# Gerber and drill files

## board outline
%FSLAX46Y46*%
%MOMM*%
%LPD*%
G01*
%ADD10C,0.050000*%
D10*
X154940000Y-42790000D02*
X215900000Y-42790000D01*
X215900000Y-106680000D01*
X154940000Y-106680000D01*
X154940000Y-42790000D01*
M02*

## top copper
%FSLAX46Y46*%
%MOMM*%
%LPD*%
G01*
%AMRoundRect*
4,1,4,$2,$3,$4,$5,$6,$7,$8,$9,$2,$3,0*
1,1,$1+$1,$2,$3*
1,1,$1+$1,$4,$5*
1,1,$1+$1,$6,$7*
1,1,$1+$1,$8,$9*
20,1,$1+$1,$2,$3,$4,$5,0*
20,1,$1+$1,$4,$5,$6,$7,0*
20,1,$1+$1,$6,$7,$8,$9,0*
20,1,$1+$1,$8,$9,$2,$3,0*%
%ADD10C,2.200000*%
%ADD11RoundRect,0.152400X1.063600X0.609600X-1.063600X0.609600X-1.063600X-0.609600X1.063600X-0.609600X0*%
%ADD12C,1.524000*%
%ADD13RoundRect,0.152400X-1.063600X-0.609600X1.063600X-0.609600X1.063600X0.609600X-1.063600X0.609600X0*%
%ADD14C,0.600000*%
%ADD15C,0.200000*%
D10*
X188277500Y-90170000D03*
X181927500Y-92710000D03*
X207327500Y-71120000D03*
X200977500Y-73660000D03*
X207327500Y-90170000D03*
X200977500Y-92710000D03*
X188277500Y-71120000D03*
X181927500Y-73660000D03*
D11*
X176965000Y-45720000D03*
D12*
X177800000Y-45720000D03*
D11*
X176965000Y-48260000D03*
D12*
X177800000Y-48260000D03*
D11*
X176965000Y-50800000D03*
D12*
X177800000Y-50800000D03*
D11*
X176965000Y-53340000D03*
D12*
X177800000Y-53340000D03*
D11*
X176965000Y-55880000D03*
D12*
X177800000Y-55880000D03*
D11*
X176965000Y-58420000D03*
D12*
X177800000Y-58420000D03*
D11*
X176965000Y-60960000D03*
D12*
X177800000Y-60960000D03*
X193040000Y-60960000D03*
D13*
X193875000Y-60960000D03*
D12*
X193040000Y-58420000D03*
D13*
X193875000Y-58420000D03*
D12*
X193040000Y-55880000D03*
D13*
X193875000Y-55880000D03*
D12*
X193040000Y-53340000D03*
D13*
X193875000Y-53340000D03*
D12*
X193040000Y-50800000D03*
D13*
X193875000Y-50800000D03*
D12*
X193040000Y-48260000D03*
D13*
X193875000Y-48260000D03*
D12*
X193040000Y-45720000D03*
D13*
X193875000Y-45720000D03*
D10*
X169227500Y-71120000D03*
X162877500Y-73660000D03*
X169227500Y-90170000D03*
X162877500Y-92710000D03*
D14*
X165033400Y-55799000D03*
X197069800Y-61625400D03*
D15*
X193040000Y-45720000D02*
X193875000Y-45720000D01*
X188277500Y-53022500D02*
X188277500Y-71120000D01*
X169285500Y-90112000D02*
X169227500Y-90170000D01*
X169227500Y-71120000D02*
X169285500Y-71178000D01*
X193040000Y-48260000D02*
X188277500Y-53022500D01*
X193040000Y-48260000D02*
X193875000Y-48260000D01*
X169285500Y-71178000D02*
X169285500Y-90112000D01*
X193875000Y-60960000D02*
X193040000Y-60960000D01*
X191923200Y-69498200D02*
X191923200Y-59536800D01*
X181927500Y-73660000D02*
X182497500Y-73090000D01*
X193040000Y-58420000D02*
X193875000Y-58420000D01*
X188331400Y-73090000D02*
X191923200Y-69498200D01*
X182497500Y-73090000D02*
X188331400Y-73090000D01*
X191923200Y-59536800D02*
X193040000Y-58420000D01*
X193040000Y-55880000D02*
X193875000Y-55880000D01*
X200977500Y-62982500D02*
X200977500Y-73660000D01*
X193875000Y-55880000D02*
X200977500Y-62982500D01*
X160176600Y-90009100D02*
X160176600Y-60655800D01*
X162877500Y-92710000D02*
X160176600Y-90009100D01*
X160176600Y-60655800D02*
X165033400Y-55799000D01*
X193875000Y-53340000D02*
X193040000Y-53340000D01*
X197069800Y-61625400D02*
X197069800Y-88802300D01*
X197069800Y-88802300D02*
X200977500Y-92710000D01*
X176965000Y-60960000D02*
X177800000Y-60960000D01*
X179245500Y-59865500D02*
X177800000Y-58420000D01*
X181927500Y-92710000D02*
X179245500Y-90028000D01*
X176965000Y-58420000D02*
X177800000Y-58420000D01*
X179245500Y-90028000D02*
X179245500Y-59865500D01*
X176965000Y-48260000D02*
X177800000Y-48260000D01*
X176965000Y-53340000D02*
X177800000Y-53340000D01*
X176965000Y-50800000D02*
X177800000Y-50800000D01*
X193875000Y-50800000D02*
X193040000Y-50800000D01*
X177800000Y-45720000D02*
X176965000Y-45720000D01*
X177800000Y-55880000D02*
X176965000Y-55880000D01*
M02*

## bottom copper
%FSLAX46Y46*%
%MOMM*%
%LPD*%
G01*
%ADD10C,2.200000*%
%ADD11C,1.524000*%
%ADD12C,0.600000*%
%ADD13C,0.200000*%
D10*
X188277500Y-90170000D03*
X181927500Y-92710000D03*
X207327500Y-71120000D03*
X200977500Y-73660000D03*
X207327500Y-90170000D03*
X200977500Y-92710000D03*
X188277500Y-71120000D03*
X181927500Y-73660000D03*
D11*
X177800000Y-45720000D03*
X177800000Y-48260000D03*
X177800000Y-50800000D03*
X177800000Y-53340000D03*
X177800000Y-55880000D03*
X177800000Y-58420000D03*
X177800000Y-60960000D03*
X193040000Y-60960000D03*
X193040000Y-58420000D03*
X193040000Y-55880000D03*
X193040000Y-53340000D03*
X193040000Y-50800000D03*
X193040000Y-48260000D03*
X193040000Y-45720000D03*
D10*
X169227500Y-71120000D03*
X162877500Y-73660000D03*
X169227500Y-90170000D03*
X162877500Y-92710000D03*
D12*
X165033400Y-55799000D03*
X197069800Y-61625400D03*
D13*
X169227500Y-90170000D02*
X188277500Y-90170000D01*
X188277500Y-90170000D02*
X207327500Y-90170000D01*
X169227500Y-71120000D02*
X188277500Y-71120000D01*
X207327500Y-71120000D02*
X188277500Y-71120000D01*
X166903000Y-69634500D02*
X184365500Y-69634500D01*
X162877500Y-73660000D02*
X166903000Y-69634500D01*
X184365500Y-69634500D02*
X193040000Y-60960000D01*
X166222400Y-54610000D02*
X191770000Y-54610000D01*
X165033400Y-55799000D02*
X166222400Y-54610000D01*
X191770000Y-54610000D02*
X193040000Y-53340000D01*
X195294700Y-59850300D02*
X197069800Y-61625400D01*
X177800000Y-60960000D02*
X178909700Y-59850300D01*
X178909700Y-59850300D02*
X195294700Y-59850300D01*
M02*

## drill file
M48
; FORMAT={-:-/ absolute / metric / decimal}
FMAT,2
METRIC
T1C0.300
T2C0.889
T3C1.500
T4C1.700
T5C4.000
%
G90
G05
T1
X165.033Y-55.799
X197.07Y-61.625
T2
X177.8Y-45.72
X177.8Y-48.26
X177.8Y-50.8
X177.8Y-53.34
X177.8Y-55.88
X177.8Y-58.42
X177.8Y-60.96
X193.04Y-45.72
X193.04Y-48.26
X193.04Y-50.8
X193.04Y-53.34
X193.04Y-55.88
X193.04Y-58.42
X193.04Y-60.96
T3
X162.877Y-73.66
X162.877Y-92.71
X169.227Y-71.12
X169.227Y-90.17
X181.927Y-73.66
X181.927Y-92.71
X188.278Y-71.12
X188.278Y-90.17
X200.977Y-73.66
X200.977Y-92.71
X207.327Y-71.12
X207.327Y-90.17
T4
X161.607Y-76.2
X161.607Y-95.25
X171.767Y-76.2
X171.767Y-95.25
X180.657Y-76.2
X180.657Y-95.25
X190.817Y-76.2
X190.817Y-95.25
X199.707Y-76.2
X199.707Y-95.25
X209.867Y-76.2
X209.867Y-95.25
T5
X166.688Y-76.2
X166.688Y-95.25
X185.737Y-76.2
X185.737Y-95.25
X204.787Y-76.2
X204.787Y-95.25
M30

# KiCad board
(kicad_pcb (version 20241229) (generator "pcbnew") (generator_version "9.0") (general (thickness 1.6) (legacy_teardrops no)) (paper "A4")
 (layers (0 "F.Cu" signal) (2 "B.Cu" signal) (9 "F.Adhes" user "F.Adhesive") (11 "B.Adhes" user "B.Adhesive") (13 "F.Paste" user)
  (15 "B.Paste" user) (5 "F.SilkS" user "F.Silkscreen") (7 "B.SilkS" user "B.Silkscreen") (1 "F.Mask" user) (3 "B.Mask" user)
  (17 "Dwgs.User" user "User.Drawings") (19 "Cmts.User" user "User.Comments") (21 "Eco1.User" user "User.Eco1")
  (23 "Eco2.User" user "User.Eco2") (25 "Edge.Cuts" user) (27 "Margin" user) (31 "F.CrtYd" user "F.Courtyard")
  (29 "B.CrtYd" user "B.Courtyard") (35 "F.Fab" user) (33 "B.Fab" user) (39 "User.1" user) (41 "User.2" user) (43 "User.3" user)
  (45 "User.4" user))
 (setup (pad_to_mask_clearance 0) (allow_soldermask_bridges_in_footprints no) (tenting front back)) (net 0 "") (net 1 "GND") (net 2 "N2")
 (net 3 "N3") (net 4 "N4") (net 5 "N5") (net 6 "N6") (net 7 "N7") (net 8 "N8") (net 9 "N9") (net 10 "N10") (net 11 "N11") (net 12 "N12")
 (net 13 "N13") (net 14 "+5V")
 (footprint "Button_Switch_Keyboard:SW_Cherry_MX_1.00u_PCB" (layer "F.Cu") (at 188.2775 90.17)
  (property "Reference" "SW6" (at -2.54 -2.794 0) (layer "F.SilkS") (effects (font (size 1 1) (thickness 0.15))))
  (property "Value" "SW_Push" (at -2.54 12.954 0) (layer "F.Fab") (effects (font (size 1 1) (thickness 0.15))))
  (pad "" np_thru_hole circle (at -7.62 5.08) (size 1.7 1.7) (drill 1.7) (layers "*.Cu" "*.Mask"))
  (pad "" np_thru_hole circle (at -2.54 5.08) (size 4 4) (drill 4) (layers "*.Cu" "*.Mask"))
  (pad "" np_thru_hole circle (at 2.54 5.08) (size 1.7 1.7) (drill 1.7) (layers "*.Cu" "*.Mask"))
  (pad "1" thru_hole circle (at 0 0) (size 2.2 2.2) (drill 1.5) (layers "*.Cu" "*.Mask") (remove_unused_layers no) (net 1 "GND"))
  (pad "2" thru_hole circle (at -6.35 2.54) (size 2.2 2.2) (drill 1.5) (layers "*.Cu" "*.Mask") (remove_unused_layers no) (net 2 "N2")))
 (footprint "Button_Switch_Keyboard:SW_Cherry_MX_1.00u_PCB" (layer "F.Cu") (at 207.3275 71.12)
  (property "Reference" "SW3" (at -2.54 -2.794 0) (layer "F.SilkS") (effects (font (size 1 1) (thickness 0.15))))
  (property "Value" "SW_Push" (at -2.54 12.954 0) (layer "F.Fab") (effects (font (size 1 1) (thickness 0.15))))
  (pad "" np_thru_hole circle (at -7.62 5.08) (size 1.7 1.7) (drill 1.7) (layers "*.Cu" "*.Mask"))
  (pad "" np_thru_hole circle (at -2.54 5.08) (size 4 4) (drill 4) (layers "*.Cu" "*.Mask"))
  (pad "" np_thru_hole circle (at 2.54 5.08) (size 1.7 1.7) (drill 1.7) (layers "*.Cu" "*.Mask"))
  (pad "1" thru_hole circle (at 0 0) (size 2.2 2.2) (drill 1.5) (layers "*.Cu" "*.Mask") (remove_unused_layers no) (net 1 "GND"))
  (pad "2" thru_hole circle (at -6.35 2.54) (size 2.2 2.2) (drill 1.5) (layers "*.Cu" "*.Mask") (remove_unused_layers no) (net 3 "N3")))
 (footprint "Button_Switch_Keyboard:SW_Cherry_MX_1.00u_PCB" (layer "F.Cu") (at 207.3275 90.17)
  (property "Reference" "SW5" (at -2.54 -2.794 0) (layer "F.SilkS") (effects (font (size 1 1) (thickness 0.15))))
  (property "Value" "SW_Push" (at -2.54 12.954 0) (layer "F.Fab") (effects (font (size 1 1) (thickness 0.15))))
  (pad "" np_thru_hole circle (at -7.62 5.08) (size 1.7 1.7) (drill 1.7) (layers "*.Cu" "*.Mask"))
  (pad "" np_thru_hole circle (at -2.54 5.08) (size 4 4) (drill 4) (layers "*.Cu" "*.Mask"))
  (pad "" np_thru_hole circle (at 2.54 5.08) (size 1.7 1.7) (drill 1.7) (layers "*.Cu" "*.Mask"))
  (pad "1" thru_hole circle (at 0 0) (size 2.2 2.2) (drill 1.5) (layers "*.Cu" "*.Mask") (remove_unused_layers no) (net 1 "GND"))
  (pad "2" thru_hole circle (at -6.35 2.54) (size 2.2 2.2) (drill 1.5) (layers "*.Cu" "*.Mask") (remove_unused_layers no) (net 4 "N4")))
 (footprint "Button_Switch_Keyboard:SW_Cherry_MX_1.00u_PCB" (layer "F.Cu") (at 188.2775 71.12)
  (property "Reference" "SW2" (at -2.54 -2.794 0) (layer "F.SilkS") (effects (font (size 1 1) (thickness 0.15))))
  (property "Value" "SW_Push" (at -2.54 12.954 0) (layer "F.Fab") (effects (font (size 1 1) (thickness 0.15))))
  (pad "" np_thru_hole circle (at -7.62 5.08) (size 1.7 1.7) (drill 1.7) (layers "*.Cu" "*.Mask"))
  (pad "" np_thru_hole circle (at -2.54 5.08) (size 4 4) (drill 4) (layers "*.Cu" "*.Mask"))
  (pad "" np_thru_hole circle (at 2.54 5.08) (size 1.7 1.7) (drill 1.7) (layers "*.Cu" "*.Mask"))
  (pad "1" thru_hole circle (at 0 0) (size 2.2 2.2) (drill 1.5) (layers "*.Cu" "*.Mask") (remove_unused_layers no) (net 1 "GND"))
  (pad "2" thru_hole circle (at -6.35 2.54) (size 2.2 2.2) (drill 1.5) (layers "*.Cu" "*.Mask") (remove_unused_layers no) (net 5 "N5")))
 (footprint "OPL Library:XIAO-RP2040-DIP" (layer "F.Cu") (at 185.42 53.34)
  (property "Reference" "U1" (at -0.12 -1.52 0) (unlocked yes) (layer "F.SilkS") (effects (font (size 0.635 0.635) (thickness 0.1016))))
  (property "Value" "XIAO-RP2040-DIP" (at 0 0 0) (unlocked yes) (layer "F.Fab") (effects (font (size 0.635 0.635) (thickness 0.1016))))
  (pad "1" smd roundrect (at -8.455 -7.62 180) (size 2.432 1.524) (layers "F.Cu" "F.Mask") (roundrect_rratio 0.1) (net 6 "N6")
   (thermal_bridge_angle 45))
  (pad "1" thru_hole circle (at -7.62 -7.62 180) (size 1.524 1.524) (drill 0.889) (layers "*.Cu" "*.Mask") (remove_unused_layers no)
   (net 6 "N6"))
  (pad "2" smd roundrect (at -8.455 -5.08 180) (size 2.432 1.524) (layers "F.Cu" "F.Mask") (roundrect_rratio 0.1) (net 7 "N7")
   (thermal_bridge_angle 45))
  (pad "2" thru_hole circle (at -7.62 -5.08 180) (size 1.524 1.524) (drill 0.889) (layers "*.Cu" "*.Mask") (remove_unused_layers no)
   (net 7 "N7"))
  (pad "3" smd roundrect (at -8.455 -2.54 180) (size 2.432 1.524) (layers "F.Cu" "F.Mask") (roundrect_rratio 0.1) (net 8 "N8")
   (thermal_bridge_angle 45))
  (pad "3" thru_hole circle (at -7.62 -2.54 180) (size 1.524 1.524) (drill 0.889) (layers "*.Cu" "*.Mask") (remove_unused_layers no)
   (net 8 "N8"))
  (pad "4" smd roundrect (at -8.455 0 180) (size 2.432 1.524) (layers "F.Cu" "F.Mask") (roundrect_rratio 0.1) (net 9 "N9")
   (thermal_bridge_angle 45))
  (pad "4" thru_hole circle (at -7.62 0 180) (size 1.524 1.524) (drill 0.889) (layers "*.Cu" "*.Mask") (remove_unused_layers no)
   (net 9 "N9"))
  (pad "5" smd roundrect (at -8.455 2.54 180) (size 2.432 1.524) (layers "F.Cu" "F.Mask") (roundrect_rratio 0.1) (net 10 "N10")
   (thermal_bridge_angle 45))
  (pad "5" thru_hole circle (at -7.62 2.54 180) (size 1.524 1.524) (drill 0.889) (layers "*.Cu" "*.Mask") (remove_unused_layers no)
   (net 10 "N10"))
  (pad "6" smd roundrect (at -8.455 5.08 180) (size 2.432 1.524) (layers "F.Cu" "F.Mask") (roundrect_rratio 0.1) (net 2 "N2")
   (thermal_bridge_angle 45))
  (pad "6" thru_hole circle (at -7.62 5.08 180) (size 1.524 1.524) (drill 0.889) (layers "*.Cu" "*.Mask") (remove_unused_layers no)
   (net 2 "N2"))
  (pad "7" smd roundrect (at -8.455 7.62 180) (size 2.432 1.524) (layers "F.Cu" "F.Mask") (roundrect_rratio 0.1) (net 4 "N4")
   (thermal_bridge_angle 45))
  (pad "7" thru_hole circle (at -7.62 7.62 180) (size 1.524 1.524) (drill 0.889) (layers "*.Cu" "*.Mask") (remove_unused_layers no)
   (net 4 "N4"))
  (pad "8" thru_hole circle (at 7.62 7.62) (size 1.524 1.524) (drill 0.889) (layers "*.Cu" "*.Mask") (remove_unused_layers no)
   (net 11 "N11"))
  (pad "8" smd roundrect (at 8.455 7.62) (size 2.432 1.524) (layers "F.Cu" "F.Mask") (roundrect_rratio 0.1) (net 11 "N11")
   (thermal_bridge_angle 45))
  (pad "9" thru_hole circle (at 7.62 5.08) (size 1.524 1.524) (drill 0.889) (layers "*.Cu" "*.Mask") (remove_unused_layers no) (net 5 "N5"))
  (pad "9" smd roundrect (at 8.455 5.08) (size 2.432 1.524) (layers "F.Cu" "F.Mask") (roundrect_rratio 0.1) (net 5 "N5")
   (thermal_bridge_angle 45))
  (pad "10" thru_hole circle (at 7.62 2.54) (size 1.524 1.524) (drill 0.889) (layers "*.Cu" "*.Mask") (remove_unused_layers no) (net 3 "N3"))
  (pad "10" smd roundrect (at 8.455 2.54) (size 2.432 1.524) (layers "F.Cu" "F.Mask") (roundrect_rratio 0.1) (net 3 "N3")
   (thermal_bridge_angle 45))
  (pad "11" thru_hole circle (at 7.62 0) (size 1.524 1.524) (drill 0.889) (layers "*.Cu" "*.Mask") (remove_unused_layers no) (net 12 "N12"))
  (pad "11" smd roundrect (at 8.455 0) (size 2.432 1.524) (layers "F.Cu" "F.Mask") (roundrect_rratio 0.1) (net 12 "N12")
   (thermal_bridge_angle 45))
  (pad "12" thru_hole circle (at 7.62 -2.54) (size 1.524 1.524) (drill 0.889) (layers "*.Cu" "*.Mask") (remove_unused_layers no)
   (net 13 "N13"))
  (pad "12" smd roundrect (at 8.455 -2.54) (size 2.432 1.524) (layers "F.Cu" "F.Mask") (roundrect_rratio 0.1) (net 13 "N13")
   (thermal_bridge_angle 45))
  (pad "13" thru_hole circle (at 7.62 -5.08) (size 1.524 1.524) (drill 0.889) (layers "*.Cu" "*.Mask") (remove_unused_layers no)
   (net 1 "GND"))
  (pad "13" smd roundrect (at 8.455 -5.08) (size 2.432 1.524) (layers "F.Cu" "F.Mask") (roundrect_rratio 0.1) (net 1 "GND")
   (thermal_bridge_angle 45))
  (pad "14" thru_hole circle (at 7.62 -7.62) (size 1.524 1.524) (drill 0.889) (layers "*.Cu" "*.Mask") (remove_unused_layers no)
   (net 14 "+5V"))
  (pad "14" smd roundrect (at 8.455 -7.62) (size 2.432 1.524) (layers "F.Cu" "F.Mask") (roundrect_rratio 0.1) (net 14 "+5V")
   (thermal_bridge_angle 45)))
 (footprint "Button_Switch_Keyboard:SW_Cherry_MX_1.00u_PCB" (layer "F.Cu") (at 169.2275 71.12)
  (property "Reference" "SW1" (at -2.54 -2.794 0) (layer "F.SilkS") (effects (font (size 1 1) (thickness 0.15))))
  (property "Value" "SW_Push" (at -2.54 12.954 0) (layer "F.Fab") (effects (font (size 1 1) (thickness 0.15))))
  (pad "" np_thru_hole circle (at -7.62 5.08) (size 1.7 1.7) (drill 1.7) (layers "*.Cu" "*.Mask"))
  (pad "" np_thru_hole circle (at -2.54 5.08) (size 4 4) (drill 4) (layers "*.Cu" "*.Mask"))
  (pad "" np_thru_hole circle (at 2.54 5.08) (size 1.7 1.7) (drill 1.7) (layers "*.Cu" "*.Mask"))
  (pad "1" thru_hole circle (at 0 0) (size 2.2 2.2) (drill 1.5) (layers "*.Cu" "*.Mask") (remove_unused_layers no) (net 1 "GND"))
  (pad "2" thru_hole circle (at -6.35 2.54) (size 2.2 2.2) (drill 1.5) (layers "*.Cu" "*.Mask") (remove_unused_layers no) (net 11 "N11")))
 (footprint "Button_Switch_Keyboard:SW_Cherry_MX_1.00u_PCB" (layer "F.Cu") (at 169.2275 90.17)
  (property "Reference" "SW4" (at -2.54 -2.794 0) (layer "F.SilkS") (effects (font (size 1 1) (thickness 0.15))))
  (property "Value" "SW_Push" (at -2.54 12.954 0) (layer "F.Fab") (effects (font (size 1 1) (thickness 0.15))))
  (pad "" np_thru_hole circle (at -7.62 5.08) (size 1.7 1.7) (drill 1.7) (layers "*.Cu" "*.Mask"))
  (pad "" np_thru_hole circle (at -2.54 5.08) (size 4 4) (drill 4) (layers "*.Cu" "*.Mask"))
  (pad "" np_thru_hole circle (at 2.54 5.08) (size 1.7 1.7) (drill 1.7) (layers "*.Cu" "*.Mask"))
  (pad "1" thru_hole circle (at 0 0) (size 2.2 2.2) (drill 1.5) (layers "*.Cu" "*.Mask") (remove_unused_layers no) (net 1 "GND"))
  (pad "2" thru_hole circle (at -6.35 2.54) (size 2.2 2.2) (drill 1.5) (layers "*.Cu" "*.Mask") (remove_unused_layers no) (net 12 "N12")))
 (gr_rect (start 154.94 42.79) (end 215.9 106.68) (stroke (width 0.05) (type default)) (fill no) (layer "Edge.Cuts"))
 (segment (start 193.04 45.72) (end 193.875 45.72) (width 0.2) (layer "F.Cu") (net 14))
 (segment (start 188.2775 53.0225) (end 188.2775 71.12) (width 0.2) (layer "F.Cu") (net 1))
 (segment (start 169.2855 90.112) (end 169.2275 90.17) (width 0.2) (layer "F.Cu") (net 1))
 (segment (start 169.2275 71.12) (end 169.2855 71.178) (width 0.2) (layer "F.Cu") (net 1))
 (segment (start 193.04 48.26) (end 188.2775 53.0225) (width 0.2) (layer "F.Cu") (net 1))
 (segment (start 193.04 48.26) (end 193.875 48.26) (width 0.2) (layer "F.Cu") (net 1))
 (segment (start 169.2855 71.178) (end 169.2855 90.112) (width 0.2) (layer "F.Cu") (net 1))
 (segment (start 169.2275 90.17) (end 188.2775 90.17) (width 0.2) (layer "B.Cu") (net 1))
 (segment (start 188.2775 90.17) (end 207.3275 90.17) (width 0.2) (layer "B.Cu") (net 1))
 (segment (start 169.2275 71.12) (end 188.2775 71.12) (width 0.2) (layer "B.Cu") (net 1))
 (segment (start 207.3275 71.12) (end 188.2775 71.12) (width 0.2) (layer "B.Cu") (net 1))
 (segment (start 193.875 60.96) (end 193.04 60.96) (width 0.2) (layer "F.Cu") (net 11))
 (segment (start 166.903 69.6345) (end 184.3655 69.6345) (width 0.2) (layer "B.Cu") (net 11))
 (segment (start 162.8775 73.66) (end 166.903 69.6345) (width 0.2) (layer "B.Cu") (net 11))
 (segment (start 184.3655 69.6345) (end 193.04 60.96) (width 0.2) (layer "B.Cu") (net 11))
 (segment (start 191.9232 69.4982) (end 191.9232 59.5368) (width 0.2) (layer "F.Cu") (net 5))
 (segment (start 181.9275 73.66) (end 182.4975 73.09) (width 0.2) (layer "F.Cu") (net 5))
 (segment (start 193.04 58.42) (end 193.875 58.42) (width 0.2) (layer "F.Cu") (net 5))
 (segment (start 188.3314 73.09) (end 191.9232 69.4982) (width 0.2) (layer "F.Cu") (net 5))
 (segment (start 182.4975 73.09) (end 188.3314 73.09) (width 0.2) (layer "F.Cu") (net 5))
 (segment (start 191.9232 59.5368) (end 193.04 58.42) (width 0.2) (layer "F.Cu") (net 5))
 (segment (start 193.04 55.88) (end 193.875 55.88) (width 0.2) (layer "F.Cu") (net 3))
 (segment (start 200.9775 62.9825) (end 200.9775 73.66) (width 0.2) (layer "F.Cu") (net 3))
 (segment (start 193.875 55.88) (end 200.9775 62.9825) (width 0.2) (layer "F.Cu") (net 3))
 (segment (start 160.1766 90.0091) (end 160.1766 60.6558) (width 0.2) (layer "F.Cu") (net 12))
 (segment (start 162.8775 92.71) (end 160.1766 90.0091) (width 0.2) (layer "F.Cu") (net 12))
 (segment (start 160.1766 60.6558) (end 165.0334 55.799) (width 0.2) (layer "F.Cu") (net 12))
 (segment (start 193.875 53.34) (end 193.04 53.34) (width 0.2) (layer "F.Cu") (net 12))
 (via (at 165.0334 55.799) (size 0.6) (drill 0.3) (layers "F.Cu" "B.Cu") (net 12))
 (segment (start 166.2224 54.61) (end 191.77 54.61) (width 0.2) (layer "B.Cu") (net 12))
 (segment (start 165.0334 55.799) (end 166.2224 54.61) (width 0.2) (layer "B.Cu") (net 12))
 (segment (start 191.77 54.61) (end 193.04 53.34) (width 0.2) (layer "B.Cu") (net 12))
 (segment (start 197.0698 61.6254) (end 197.0698 88.8023) (width 0.2) (layer "F.Cu") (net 4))
 (segment (start 197.0698 88.8023) (end 200.9775 92.71) (width 0.2) (layer "F.Cu") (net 4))
 (segment (start 176.965 60.96) (end 177.8 60.96) (width 0.2) (layer "F.Cu") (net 4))
 (via (at 197.0698 61.6254) (size 0.6) (drill 0.3) (layers "F.Cu" "B.Cu") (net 4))
 (segment (start 195.2947 59.8503) (end 197.0698 61.6254) (width 0.2) (layer "B.Cu") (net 4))
 (segment (start 177.8 60.96) (end 178.9097 59.8503) (width 0.2) (layer "B.Cu") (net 4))
 (segment (start 178.9097 59.8503) (end 195.2947 59.8503) (width 0.2) (layer "B.Cu") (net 4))
 (segment (start 179.2455 59.8655) (end 177.8 58.42) (width 0.2) (layer "F.Cu") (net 2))
 (segment (start 181.9275 92.71) (end 179.2455 90.028) (width 0.2) (layer "F.Cu") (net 2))
 (segment (start 176.965 58.42) (end 177.8 58.42) (width 0.2) (layer "F.Cu") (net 2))
 (segment (start 179.2455 90.028) (end 179.2455 59.8655) (width 0.2) (layer "F.Cu") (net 2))
 (segment (start 176.965 48.26) (end 177.8 48.26) (width 0.2) (layer "F.Cu") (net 7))
 (segment (start 176.965 53.34) (end 177.8 53.34) (width 0.2) (layer "F.Cu") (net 9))
 (segment (start 176.965 50.8) (end 177.8 50.8) (width 0.2) (layer "F.Cu") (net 8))
 (segment (start 193.875 50.8) (end 193.04 50.8) (width 0.2) (layer "F.Cu") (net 13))
 (segment (start 177.8 45.72) (end 176.965 45.72) (width 0.2) (layer "F.Cu") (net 6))
 (segment (start 177.8 55.88) (end 176.965 55.88) (width 0.2) (layer "F.Cu") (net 10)))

